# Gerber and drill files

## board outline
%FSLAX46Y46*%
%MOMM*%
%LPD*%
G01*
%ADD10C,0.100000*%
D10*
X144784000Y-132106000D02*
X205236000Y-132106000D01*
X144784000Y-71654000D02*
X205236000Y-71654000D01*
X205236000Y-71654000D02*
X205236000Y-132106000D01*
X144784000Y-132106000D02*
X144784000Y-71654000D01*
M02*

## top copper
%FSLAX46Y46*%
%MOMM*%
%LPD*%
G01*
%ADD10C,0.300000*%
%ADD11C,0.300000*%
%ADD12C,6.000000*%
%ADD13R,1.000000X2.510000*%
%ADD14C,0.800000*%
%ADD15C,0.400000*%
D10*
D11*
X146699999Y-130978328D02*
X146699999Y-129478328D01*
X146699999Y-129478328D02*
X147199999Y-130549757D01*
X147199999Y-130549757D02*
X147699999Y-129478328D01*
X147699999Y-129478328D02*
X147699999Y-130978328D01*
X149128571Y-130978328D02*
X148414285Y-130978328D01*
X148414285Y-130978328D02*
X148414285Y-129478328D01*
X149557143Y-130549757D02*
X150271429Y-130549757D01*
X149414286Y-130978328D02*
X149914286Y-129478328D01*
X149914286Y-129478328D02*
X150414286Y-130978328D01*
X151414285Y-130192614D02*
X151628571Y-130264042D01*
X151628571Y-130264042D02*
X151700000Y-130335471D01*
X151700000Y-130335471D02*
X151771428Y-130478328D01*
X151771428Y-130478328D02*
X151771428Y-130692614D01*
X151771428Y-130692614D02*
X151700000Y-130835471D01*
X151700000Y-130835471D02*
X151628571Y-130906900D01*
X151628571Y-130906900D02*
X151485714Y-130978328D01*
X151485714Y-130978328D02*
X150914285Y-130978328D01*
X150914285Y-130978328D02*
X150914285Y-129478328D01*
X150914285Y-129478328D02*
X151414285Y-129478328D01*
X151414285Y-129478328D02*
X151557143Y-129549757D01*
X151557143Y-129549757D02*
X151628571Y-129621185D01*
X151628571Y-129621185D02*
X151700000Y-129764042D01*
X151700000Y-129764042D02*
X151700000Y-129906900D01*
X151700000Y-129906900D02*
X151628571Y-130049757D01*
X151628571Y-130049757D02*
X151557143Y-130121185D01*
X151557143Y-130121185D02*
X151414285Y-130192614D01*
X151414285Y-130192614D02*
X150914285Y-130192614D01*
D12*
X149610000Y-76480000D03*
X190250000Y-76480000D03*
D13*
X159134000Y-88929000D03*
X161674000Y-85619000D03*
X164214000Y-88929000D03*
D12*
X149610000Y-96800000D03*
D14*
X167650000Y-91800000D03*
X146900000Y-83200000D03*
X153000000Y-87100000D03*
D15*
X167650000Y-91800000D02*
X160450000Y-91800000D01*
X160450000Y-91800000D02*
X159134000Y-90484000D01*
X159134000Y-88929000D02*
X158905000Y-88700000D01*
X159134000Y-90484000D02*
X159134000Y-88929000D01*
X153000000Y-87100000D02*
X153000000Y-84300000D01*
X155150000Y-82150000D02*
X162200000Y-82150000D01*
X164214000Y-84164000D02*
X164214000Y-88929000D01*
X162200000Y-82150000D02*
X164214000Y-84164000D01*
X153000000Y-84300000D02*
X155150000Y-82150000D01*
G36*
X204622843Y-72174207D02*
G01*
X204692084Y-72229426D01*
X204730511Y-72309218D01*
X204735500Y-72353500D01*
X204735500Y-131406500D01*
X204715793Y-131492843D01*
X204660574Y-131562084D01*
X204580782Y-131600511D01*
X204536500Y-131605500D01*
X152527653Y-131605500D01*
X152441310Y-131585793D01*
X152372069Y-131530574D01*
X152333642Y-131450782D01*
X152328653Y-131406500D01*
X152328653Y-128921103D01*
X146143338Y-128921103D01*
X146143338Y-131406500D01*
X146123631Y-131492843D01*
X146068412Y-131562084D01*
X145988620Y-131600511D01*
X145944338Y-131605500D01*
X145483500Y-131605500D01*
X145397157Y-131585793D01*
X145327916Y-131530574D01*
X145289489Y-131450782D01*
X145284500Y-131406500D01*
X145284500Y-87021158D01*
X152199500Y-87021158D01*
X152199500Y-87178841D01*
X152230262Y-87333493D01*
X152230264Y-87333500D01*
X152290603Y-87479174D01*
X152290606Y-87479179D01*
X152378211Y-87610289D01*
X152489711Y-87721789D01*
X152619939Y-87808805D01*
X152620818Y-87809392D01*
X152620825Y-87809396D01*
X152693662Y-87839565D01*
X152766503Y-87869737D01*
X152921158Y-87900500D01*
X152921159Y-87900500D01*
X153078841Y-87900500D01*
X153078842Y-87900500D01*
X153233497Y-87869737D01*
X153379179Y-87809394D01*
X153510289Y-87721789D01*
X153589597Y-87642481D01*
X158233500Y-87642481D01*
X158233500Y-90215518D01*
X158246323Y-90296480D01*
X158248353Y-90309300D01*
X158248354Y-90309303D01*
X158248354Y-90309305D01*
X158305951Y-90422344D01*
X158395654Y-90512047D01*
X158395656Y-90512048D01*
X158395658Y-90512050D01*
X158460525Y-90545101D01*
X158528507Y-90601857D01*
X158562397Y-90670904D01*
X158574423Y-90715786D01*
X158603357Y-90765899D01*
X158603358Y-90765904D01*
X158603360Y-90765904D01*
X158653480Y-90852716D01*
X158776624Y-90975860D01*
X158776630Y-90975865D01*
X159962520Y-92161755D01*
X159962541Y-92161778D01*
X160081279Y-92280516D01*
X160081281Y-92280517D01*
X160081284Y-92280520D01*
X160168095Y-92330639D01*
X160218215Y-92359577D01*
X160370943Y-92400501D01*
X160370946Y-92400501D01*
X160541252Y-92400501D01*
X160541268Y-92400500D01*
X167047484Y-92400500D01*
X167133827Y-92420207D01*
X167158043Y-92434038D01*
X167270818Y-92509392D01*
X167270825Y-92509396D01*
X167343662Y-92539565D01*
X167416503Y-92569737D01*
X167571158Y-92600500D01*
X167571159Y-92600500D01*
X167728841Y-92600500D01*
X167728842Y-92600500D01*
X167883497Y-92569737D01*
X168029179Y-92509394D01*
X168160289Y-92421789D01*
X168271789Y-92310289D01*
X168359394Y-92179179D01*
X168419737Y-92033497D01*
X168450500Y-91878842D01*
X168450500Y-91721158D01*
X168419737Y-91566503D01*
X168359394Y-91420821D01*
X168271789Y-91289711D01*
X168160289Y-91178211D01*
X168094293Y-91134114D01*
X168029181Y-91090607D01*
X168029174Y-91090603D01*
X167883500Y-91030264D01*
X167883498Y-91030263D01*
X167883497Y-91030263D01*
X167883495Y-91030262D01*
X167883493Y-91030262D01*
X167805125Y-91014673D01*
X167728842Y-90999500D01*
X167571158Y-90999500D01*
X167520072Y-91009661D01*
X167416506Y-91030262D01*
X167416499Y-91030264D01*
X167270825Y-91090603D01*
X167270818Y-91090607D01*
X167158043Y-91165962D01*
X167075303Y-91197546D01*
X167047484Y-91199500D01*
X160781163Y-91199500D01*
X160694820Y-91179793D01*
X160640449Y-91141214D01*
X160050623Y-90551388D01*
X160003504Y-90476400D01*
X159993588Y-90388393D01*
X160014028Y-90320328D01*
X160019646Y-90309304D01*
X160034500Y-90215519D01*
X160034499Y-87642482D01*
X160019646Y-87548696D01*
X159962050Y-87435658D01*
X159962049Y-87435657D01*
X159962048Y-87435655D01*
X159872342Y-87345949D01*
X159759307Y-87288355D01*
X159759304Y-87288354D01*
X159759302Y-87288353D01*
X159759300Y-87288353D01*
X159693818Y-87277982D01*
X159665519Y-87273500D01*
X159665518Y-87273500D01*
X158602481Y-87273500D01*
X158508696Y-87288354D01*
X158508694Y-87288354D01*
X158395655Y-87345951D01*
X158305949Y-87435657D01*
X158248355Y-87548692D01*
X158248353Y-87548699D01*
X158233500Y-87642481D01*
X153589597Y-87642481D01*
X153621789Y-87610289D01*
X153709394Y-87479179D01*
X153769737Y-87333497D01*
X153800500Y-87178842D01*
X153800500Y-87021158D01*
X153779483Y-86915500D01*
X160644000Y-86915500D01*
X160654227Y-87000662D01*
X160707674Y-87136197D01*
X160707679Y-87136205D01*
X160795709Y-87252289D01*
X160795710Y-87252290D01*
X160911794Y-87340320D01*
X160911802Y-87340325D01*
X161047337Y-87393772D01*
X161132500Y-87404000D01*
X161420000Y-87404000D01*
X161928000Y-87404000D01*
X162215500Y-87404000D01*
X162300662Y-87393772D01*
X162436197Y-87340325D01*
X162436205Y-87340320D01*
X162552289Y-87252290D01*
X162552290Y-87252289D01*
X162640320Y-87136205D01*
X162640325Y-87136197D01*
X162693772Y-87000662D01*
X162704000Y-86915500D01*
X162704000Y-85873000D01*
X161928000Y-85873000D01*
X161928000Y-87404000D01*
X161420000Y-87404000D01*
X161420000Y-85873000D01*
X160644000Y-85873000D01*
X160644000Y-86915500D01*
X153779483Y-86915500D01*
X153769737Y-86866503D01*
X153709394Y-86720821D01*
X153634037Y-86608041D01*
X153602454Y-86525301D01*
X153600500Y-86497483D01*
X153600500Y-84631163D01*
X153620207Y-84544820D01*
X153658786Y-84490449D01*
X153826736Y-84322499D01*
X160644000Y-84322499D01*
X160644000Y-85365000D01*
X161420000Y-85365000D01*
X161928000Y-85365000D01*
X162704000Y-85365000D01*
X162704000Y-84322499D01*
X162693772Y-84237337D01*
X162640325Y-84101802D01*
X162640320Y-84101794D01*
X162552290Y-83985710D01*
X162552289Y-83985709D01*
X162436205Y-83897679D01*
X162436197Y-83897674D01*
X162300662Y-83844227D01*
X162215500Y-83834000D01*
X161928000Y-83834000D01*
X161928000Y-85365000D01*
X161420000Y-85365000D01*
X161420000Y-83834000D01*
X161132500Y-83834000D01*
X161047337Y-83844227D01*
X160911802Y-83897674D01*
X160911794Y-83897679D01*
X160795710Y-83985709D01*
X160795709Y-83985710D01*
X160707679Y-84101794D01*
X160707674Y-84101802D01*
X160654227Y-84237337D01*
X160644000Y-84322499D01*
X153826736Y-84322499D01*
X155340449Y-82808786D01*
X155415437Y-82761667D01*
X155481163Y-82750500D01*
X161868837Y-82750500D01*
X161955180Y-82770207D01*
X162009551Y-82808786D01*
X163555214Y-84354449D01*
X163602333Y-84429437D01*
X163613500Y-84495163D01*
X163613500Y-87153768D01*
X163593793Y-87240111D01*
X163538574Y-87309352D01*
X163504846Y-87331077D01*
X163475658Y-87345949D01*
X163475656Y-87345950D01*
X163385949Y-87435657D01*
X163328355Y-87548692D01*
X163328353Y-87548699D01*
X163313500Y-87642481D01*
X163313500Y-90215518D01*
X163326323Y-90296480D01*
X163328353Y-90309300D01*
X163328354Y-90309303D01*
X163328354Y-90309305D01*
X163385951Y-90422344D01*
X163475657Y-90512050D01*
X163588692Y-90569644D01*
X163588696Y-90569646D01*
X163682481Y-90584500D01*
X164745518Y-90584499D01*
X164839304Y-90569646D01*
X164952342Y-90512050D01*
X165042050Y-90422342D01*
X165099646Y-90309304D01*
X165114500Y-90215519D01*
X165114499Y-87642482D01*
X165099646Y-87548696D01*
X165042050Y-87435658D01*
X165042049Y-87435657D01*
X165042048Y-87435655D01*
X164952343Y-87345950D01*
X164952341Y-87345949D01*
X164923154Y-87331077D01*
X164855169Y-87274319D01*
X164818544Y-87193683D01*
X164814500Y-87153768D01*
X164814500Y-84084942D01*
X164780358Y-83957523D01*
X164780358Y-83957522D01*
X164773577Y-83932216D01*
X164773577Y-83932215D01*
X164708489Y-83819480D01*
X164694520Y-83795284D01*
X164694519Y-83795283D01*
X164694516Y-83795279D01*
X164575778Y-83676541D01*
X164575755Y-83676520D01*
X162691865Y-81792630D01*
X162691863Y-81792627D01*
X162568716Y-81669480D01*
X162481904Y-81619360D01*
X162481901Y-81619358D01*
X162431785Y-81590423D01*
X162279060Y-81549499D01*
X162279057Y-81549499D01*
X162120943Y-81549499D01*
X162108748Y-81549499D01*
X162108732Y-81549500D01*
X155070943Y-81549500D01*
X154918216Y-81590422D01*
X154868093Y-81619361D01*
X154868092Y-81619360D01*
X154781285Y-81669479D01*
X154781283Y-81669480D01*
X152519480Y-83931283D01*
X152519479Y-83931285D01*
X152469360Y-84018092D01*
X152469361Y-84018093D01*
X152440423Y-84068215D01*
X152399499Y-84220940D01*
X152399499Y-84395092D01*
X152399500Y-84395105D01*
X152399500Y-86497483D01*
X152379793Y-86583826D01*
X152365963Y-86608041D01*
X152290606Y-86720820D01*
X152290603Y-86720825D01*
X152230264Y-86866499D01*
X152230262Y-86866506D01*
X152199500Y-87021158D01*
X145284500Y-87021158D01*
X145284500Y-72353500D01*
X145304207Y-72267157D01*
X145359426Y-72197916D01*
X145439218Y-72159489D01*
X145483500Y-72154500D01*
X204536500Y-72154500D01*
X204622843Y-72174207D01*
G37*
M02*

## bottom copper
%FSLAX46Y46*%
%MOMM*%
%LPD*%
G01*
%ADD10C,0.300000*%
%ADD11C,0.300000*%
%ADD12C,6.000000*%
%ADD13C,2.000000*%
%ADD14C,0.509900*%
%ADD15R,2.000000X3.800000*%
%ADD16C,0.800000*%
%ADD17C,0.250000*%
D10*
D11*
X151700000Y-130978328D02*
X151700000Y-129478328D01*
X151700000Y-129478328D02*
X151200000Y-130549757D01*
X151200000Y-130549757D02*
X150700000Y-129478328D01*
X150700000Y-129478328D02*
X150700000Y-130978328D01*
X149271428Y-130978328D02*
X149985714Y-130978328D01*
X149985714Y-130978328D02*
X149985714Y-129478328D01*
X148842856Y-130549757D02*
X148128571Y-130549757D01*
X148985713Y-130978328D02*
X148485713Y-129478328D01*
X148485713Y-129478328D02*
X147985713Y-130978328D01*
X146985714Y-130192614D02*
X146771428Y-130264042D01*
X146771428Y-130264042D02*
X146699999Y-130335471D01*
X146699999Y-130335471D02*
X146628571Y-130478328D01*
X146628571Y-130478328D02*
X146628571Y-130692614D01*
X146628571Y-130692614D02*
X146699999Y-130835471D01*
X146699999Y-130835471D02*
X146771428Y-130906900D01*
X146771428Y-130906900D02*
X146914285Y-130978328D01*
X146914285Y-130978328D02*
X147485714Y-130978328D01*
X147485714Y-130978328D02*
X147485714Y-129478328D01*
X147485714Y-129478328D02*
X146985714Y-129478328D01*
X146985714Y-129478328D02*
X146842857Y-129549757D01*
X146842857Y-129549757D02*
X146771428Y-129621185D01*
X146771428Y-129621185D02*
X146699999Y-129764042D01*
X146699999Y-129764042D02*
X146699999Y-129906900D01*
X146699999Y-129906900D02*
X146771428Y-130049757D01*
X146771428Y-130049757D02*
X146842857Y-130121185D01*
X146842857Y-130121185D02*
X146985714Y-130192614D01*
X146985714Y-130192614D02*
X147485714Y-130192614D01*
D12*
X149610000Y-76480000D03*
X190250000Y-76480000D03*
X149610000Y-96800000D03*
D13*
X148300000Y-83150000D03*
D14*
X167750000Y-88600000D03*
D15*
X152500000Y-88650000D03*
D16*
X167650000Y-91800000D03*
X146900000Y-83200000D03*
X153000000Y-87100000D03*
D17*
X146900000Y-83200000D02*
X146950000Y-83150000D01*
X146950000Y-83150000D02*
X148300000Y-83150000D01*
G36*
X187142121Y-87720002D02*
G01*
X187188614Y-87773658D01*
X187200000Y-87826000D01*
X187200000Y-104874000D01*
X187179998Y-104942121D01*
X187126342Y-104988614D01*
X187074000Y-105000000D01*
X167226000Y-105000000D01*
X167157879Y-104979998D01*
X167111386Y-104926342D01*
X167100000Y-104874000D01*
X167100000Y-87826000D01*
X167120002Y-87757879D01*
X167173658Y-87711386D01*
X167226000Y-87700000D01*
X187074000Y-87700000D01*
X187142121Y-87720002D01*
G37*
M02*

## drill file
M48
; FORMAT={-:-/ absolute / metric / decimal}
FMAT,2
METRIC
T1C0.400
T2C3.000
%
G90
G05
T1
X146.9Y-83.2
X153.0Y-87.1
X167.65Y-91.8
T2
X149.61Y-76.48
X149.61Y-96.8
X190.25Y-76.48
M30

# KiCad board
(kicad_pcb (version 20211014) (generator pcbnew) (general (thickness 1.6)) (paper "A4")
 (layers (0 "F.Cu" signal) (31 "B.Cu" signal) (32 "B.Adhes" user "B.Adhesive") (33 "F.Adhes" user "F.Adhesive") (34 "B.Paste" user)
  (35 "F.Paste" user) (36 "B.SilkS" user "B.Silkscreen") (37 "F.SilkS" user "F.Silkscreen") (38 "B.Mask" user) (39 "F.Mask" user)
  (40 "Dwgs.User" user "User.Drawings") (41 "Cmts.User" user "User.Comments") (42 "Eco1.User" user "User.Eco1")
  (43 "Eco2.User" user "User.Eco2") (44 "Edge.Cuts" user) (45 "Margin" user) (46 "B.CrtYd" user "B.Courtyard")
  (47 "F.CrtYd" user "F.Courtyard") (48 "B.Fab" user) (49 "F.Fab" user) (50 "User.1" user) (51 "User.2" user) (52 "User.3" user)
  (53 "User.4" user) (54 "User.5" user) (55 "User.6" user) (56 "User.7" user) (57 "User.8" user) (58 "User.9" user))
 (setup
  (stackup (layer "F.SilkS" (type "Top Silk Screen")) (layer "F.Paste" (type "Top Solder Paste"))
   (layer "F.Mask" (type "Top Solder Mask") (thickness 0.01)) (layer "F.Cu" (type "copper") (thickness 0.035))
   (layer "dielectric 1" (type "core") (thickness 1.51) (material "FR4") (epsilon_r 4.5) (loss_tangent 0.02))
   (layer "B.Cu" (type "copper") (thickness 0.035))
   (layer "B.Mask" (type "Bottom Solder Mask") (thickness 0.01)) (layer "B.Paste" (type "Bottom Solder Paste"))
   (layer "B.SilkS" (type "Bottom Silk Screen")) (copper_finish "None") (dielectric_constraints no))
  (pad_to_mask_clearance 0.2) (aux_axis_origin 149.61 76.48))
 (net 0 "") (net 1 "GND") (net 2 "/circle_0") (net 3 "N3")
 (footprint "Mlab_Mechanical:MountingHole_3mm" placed (layer "F.Cu") (at 149.61 76.48)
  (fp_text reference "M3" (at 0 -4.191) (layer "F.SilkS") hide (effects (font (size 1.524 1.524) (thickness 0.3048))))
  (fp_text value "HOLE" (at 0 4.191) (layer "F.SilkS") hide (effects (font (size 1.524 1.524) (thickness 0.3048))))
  (pad "1" thru_hole circle (at 0 0) (size 6 6) (drill 3) (layers *.Cu *.Mask) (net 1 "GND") (clearance 1) (zone_connect 2)))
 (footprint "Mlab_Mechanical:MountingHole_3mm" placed (layer "F.Cu") (at 190.25 76.48)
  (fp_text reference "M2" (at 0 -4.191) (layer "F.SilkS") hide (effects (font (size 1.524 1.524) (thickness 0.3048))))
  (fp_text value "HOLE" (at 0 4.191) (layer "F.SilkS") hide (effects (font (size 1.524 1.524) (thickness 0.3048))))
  (pad "1" thru_hole circle (at 0 0) (size 6 6) (drill 3) (layers *.Cu *.Mask) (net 1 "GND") (clearance 1) (zone_connect 2)))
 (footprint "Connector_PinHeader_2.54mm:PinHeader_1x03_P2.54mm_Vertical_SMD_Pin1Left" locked (layer "F.Cu") (at 161.674 87.274 90)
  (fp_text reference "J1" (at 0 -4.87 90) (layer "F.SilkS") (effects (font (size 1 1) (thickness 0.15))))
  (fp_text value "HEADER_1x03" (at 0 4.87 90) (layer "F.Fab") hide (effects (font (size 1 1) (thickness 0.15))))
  (pad "1" smd rect locked (at -1.655 -2.54 90) (size 2.51 1) (layers "F.Cu" "F.Paste" "F.Mask") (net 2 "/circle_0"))
  (pad "2" smd rect locked (at 1.655 0 90) (size 2.51 1) (layers "F.Cu" "F.Paste" "F.Mask") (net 1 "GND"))
  (pad "3" smd rect locked (at -1.655 2.54 90) (size 2.51 1) (layers "F.Cu" "F.Paste" "F.Mask") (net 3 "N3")))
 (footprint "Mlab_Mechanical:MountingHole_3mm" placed (layer "F.Cu") (at 149.61 96.8)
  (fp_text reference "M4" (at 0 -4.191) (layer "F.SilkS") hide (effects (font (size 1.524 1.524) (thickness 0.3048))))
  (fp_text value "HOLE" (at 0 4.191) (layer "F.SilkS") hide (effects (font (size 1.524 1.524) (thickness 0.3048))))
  (pad "1" thru_hole circle (at 0 0) (size 6 6) (drill 3) (layers *.Cu *.Mask) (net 1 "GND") (clearance 1) (zone_connect 2)))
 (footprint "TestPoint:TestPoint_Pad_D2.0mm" (layer "B.Cu") (at 148.3 83.15 180) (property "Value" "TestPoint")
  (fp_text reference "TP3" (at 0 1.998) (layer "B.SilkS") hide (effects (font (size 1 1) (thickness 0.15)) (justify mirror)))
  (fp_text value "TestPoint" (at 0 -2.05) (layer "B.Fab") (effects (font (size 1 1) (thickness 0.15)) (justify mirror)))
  (pad "1" smd circle (at 0 0 180) (size 2 2) (layers "B.Cu" "B.Mask") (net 1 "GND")))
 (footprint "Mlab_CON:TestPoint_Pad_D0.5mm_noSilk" (layer "B.Cu") (at 167.75 88.6 180) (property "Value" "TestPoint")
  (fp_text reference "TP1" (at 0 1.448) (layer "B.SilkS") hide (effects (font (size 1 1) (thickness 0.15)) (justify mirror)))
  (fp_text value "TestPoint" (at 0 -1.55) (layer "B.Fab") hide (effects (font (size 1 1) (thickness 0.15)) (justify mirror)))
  (pad "1" smd circle (at 0 0 180) (size 0.5099 0.5099) (layers "B.Cu" "B.Mask") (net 2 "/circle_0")))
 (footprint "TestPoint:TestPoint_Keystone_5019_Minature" (layer "B.Cu") (at 152.5 88.65 90) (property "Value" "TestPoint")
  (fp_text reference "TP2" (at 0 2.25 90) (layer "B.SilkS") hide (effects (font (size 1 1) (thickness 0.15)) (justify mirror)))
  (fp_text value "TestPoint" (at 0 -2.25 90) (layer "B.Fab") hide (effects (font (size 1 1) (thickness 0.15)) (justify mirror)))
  (pad "1" smd rect (at 0 0 90) (size 3.8 2) (layers "B.Cu" "B.Paste" "B.Mask") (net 3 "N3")))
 (gr_line (start 144.784 132.106) (end 205.236 132.106) (layer "Edge.Cuts") (width 0.1))
 (gr_line (start 144.784 71.654) (end 205.236 71.654) (layer "Edge.Cuts") (width 0.1))
 (gr_line (start 205.236 71.654) (end 205.236 132.106) (layer "Edge.Cuts") (width 0.1))
 (gr_line (start 144.784 132.106) (end 144.784 71.654) (layer "Edge.Cuts") (width 0.1))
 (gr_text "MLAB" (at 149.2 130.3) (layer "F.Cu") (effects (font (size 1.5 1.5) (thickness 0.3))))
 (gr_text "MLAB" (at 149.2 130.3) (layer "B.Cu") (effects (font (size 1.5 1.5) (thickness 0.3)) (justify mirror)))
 (segment (start 167.65 91.8) (end 160.45 91.8) (width 0.4) (layer "F.Cu") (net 2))
 (segment (start 160.45 91.8) (end 159.134 90.484) (width 0.4) (layer "F.Cu") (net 2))
 (segment (start 159.134 88.929) (end 158.905 88.7) (width 0.4) (layer "F.Cu") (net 2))
 (segment (start 159.134 90.484) (end 159.134 88.929) (width 0.4) (layer "F.Cu") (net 2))
 (via (at 167.65 91.8) (size 0.8) (drill 0.4) (layers "F.Cu" "B.Cu") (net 2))
 (via (at 146.9 83.2) (size 0.8) (drill 0.4) (layers "F.Cu" "B.Cu") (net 1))
 (segment (start 146.9 83.2) (end 146.95 83.15) (width 0.25) (layer "B.Cu") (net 1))
 (segment (start 146.95 83.15) (end 148.3 83.15) (width 0.25) (layer "B.Cu") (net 1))
 (segment (start 153 87.1) (end 153 84.3) (width 0.4) (layer "F.Cu") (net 3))
 (segment (start 155.15 82.15) (end 162.2 82.15) (width 0.4) (layer "F.Cu") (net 3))
 (segment (start 164.214 84.164) (end 164.214 88.929) (width 0.4) (layer "F.Cu") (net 3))
 (segment (start 162.2 82.15) (end 164.214 84.164) (width 0.4) (layer "F.Cu") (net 3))
 (segment (start 153 84.3) (end 155.15 82.15) (width 0.4) (layer "F.Cu") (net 3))
 (via (at 153 87.1) (size 0.8) (drill 0.4) (layers "F.Cu" "B.Cu") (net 3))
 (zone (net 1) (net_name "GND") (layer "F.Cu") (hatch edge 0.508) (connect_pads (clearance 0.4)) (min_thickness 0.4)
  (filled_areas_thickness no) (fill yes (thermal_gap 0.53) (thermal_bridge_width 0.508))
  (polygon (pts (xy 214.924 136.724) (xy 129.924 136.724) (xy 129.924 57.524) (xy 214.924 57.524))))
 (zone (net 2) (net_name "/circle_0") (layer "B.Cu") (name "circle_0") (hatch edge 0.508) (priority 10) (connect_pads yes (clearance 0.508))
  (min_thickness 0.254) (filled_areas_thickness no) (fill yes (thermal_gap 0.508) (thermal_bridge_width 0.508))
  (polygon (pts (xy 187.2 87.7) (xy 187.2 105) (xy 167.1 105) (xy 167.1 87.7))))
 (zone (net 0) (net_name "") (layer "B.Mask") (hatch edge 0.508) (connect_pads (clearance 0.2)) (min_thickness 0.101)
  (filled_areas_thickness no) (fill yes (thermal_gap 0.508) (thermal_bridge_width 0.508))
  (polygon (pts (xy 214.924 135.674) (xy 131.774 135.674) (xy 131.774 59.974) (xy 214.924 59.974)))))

